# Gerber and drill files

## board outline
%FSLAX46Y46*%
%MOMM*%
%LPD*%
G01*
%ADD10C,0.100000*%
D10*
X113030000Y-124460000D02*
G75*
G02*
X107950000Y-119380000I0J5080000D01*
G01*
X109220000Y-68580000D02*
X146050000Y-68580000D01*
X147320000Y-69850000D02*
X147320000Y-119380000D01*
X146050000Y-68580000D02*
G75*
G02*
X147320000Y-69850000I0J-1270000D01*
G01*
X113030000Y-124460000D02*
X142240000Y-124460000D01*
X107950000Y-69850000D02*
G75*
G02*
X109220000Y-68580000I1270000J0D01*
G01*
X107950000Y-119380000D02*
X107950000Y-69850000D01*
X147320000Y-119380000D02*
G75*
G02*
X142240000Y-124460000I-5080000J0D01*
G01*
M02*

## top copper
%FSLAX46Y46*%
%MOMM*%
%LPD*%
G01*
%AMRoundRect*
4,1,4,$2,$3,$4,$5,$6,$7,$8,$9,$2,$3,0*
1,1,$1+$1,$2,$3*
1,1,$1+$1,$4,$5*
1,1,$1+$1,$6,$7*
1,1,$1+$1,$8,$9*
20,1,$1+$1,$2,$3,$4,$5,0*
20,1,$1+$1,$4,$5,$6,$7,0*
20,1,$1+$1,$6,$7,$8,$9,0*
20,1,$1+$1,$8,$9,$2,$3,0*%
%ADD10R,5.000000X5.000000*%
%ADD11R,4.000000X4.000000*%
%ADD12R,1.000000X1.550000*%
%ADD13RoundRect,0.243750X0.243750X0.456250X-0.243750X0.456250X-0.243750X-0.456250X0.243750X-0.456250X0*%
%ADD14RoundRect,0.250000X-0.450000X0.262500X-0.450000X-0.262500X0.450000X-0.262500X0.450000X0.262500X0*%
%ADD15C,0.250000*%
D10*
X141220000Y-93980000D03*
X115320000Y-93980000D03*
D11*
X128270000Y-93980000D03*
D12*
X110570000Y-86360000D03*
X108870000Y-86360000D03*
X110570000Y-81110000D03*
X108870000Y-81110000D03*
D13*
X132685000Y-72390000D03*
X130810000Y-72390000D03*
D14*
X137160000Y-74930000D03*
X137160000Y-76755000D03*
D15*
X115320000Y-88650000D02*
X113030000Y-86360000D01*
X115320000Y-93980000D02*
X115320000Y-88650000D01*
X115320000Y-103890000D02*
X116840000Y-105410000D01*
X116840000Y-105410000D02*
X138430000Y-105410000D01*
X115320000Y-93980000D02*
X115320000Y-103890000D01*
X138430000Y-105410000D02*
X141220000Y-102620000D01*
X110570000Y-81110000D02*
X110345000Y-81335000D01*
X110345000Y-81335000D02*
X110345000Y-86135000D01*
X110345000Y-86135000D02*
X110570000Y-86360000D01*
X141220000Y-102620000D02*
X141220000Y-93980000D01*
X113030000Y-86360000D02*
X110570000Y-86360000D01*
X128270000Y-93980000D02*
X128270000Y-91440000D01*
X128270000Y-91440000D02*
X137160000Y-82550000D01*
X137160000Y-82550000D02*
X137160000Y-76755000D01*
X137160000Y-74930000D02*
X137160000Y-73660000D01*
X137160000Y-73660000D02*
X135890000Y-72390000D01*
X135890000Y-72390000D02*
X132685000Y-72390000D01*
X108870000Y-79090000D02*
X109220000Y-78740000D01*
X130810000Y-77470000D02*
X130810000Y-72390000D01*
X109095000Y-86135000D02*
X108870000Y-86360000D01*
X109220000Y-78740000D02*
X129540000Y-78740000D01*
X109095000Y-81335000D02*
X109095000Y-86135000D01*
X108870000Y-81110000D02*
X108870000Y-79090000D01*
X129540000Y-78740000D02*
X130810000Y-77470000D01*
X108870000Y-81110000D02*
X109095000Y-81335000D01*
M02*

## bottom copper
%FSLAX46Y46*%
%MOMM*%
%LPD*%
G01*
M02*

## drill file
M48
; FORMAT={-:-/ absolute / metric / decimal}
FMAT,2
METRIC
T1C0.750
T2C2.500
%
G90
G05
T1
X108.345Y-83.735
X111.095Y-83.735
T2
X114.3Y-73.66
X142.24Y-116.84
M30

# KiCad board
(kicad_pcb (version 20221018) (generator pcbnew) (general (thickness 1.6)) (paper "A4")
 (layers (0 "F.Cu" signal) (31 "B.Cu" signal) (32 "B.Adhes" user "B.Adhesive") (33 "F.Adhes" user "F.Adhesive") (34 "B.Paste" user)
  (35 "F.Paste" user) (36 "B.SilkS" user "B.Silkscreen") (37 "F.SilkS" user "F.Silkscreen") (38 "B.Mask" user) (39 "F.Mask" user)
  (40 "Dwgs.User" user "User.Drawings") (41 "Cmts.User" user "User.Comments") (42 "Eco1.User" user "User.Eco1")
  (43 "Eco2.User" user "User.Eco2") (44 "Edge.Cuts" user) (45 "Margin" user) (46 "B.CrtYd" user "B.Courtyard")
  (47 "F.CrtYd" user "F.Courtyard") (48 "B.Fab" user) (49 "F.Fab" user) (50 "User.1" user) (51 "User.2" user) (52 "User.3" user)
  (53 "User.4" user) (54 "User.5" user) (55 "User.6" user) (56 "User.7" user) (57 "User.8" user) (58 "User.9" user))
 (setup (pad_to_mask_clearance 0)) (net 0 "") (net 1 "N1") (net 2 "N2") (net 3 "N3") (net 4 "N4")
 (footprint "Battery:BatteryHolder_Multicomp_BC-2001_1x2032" (layer "F.Cu") (at 128.27 93.98 180)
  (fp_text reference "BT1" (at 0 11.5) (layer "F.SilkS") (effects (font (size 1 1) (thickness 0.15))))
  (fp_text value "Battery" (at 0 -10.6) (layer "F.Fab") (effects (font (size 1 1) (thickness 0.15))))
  (pad "1" smd rect (at -12.95 0 180) (size 5 5) (layers "F.Cu" "F.Paste" "F.Mask") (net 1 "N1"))
  (pad "1" smd rect (at 12.95 0 180) (size 5 5) (layers "F.Cu" "F.Paste" "F.Mask") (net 1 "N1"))
  (pad "2" smd rect (at 0 0 180) (size 4 4) (layers "F.Cu" "F.Paste" "F.Mask") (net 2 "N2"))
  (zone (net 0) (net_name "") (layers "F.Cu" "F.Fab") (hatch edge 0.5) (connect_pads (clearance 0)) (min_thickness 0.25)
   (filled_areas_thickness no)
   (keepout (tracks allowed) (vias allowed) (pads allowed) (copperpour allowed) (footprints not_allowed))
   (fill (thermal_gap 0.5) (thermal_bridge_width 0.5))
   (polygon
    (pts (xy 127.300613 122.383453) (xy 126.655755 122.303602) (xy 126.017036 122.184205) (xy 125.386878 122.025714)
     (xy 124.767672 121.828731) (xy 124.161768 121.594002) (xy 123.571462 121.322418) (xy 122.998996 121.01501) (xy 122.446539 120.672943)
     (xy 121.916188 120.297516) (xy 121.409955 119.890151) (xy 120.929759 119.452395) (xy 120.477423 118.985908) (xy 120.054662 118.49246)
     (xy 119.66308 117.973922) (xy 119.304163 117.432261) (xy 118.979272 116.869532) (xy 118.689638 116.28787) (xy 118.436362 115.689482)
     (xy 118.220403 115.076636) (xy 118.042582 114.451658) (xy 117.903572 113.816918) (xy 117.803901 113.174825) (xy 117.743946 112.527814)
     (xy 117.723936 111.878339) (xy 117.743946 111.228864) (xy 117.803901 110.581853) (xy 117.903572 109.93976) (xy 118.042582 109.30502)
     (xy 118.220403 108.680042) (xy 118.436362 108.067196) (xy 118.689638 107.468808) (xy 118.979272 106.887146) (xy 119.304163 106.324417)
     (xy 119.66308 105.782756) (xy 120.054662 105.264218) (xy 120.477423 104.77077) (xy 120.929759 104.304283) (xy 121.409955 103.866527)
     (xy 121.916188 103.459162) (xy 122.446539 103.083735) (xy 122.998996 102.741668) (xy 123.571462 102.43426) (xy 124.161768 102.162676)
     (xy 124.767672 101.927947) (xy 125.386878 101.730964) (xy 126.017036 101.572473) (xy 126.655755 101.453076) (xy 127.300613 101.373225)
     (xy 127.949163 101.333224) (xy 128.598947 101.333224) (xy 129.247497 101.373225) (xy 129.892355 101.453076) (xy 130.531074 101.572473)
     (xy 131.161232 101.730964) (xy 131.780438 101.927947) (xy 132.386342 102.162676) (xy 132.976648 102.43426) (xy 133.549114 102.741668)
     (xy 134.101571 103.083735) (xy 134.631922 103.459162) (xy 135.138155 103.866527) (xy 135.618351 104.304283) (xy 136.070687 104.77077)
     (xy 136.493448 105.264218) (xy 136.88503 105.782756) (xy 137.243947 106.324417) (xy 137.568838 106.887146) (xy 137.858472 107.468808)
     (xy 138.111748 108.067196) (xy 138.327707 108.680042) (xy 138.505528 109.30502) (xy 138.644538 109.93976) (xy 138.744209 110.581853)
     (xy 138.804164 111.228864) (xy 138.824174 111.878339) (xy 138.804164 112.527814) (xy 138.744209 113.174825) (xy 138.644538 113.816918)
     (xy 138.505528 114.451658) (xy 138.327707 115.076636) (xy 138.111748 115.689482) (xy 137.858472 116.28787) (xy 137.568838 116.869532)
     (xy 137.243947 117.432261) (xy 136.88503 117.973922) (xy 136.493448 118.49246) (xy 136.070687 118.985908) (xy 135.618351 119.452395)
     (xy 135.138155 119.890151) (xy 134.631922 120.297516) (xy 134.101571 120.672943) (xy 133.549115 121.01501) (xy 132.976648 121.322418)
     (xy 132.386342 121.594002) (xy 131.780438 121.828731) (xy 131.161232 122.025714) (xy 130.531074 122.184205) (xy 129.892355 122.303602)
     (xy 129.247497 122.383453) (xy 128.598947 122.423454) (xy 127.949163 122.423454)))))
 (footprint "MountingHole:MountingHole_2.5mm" (layer "F.Cu") (at 142.24 116.84)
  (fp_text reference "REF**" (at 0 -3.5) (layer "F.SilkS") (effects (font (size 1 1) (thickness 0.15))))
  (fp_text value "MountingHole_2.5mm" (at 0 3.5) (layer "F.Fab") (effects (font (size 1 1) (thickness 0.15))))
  (pad "" np_thru_hole circle (at 0 0) (size 2.5 2.5) (drill 2.5) (layers "*.Cu" "*.Mask")))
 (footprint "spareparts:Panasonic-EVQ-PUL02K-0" (layer "F.Cu") (at 109.22 83.735 -90)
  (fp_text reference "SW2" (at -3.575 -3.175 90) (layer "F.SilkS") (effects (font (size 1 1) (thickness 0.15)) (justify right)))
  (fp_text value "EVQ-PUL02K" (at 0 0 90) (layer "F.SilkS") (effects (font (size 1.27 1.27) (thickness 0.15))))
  (pad "" np_thru_hole circle (at 0 -1.875 270) (size 0.75 0.75) (drill 0.75) (layers "*.Cu" "*.Mask"))
  (pad "" np_thru_hole circle (at 0 0.875 270) (size 0.75 0.75) (drill 0.75) (layers "*.Cu" "*.Mask"))
  (pad "1" smd rect (at 2.625 -1.35 270) (size 1.55 1) (layers "F.Cu" "F.Paste" "F.Mask") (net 1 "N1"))
  (pad "2" smd rect (at 2.625 0.35 270) (size 1.55 1) (layers "F.Cu" "F.Paste" "F.Mask") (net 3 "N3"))
  (pad "3" smd rect (at -2.625 -1.35 270) (size 1.55 1) (layers "F.Cu" "F.Paste" "F.Mask") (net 1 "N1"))
  (pad "4" smd rect (at -2.625 0.35 270) (size 1.55 1) (layers "F.Cu" "F.Paste" "F.Mask") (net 3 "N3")))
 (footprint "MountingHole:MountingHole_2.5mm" (layer "F.Cu") (at 114.3 73.66)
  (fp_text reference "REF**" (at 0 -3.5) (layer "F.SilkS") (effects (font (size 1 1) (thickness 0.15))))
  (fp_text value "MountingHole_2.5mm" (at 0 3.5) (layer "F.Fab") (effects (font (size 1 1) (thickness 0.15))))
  (pad "" np_thru_hole circle (at 0 0) (size 2.5 2.5) (drill 2.5) (layers "*.Cu" "*.Mask")))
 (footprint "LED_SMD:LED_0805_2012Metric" (layer "F.Cu") (at 131.7475 72.39 180)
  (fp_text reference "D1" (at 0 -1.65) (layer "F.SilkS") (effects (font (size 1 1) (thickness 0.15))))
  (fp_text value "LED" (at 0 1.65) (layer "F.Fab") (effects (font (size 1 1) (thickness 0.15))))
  (pad "1" smd roundrect (at -0.9375 0 180) (size 0.975 1.4) (layers "F.Cu" "F.Paste" "F.Mask") (roundrect_rratio 0.25) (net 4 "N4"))
  (pad "2" smd roundrect (at 0.9375 0 180) (size 0.975 1.4) (layers "F.Cu" "F.Paste" "F.Mask") (roundrect_rratio 0.25) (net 3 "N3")))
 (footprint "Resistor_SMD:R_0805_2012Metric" (layer "F.Cu") (at 137.16 75.8425 -90)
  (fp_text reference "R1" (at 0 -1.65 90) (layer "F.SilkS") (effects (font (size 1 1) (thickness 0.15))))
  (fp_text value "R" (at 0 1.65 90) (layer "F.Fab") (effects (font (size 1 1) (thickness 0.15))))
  (pad "1" smd roundrect (at -0.9125 0 270) (size 1.025 1.4) (layers "F.Cu" "F.Paste" "F.Mask") (roundrect_rratio 0.243902) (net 4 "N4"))
  (pad "2" smd roundrect (at 0.9125 0 270) (size 1.025 1.4) (layers "F.Cu" "F.Paste" "F.Mask") (roundrect_rratio 0.243902) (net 2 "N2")))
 (gr_arc (start 113.03 124.46) (mid 109.437898 122.972102) (end 107.95 119.38) (stroke (width 0.1) (type default)) (layer "Edge.Cuts"))
 (gr_line (start 109.22 68.58) (end 146.05 68.58) (stroke (width 0.1) (type default)) (layer "Edge.Cuts"))
 (gr_line (start 147.32 69.85) (end 147.32 119.38) (stroke (width 0.1) (type default)) (layer "Edge.Cuts"))
 (gr_arc (start 146.05 68.58) (mid 146.948026 68.951974) (end 147.32 69.85) (stroke (width 0.1) (type default)) (layer "Edge.Cuts"))
 (gr_line (start 113.03 124.46) (end 142.24 124.46) (stroke (width 0.1) (type default)) (layer "Edge.Cuts"))
 (gr_arc (start 107.95 69.85) (mid 108.321974 68.951974) (end 109.22 68.58) (stroke (width 0.1) (type default)) (layer "Edge.Cuts"))
 (gr_line (start 107.95 119.38) (end 107.95 69.85) (stroke (width 0.1) (type default)) (layer "Edge.Cuts"))
 (gr_arc (start 147.32 119.38) (mid 145.832102 122.972102) (end 142.24 124.46) (stroke (width 0.1) (type default)) (layer "Edge.Cuts"))
 (segment (start 115.32 88.65) (end 113.03 86.36) (width 0.25) (layer "F.Cu") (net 1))
 (segment (start 115.32 93.98) (end 115.32 88.65) (width 0.25) (layer "F.Cu") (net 1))
 (segment (start 115.32 103.89) (end 116.84 105.41) (width 0.25) (layer "F.Cu") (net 1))
 (segment (start 116.84 105.41) (end 138.43 105.41) (width 0.25) (layer "F.Cu") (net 1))
 (segment (start 115.32 93.98) (end 115.32 103.89) (width 0.25) (layer "F.Cu") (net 1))
 (segment (start 138.43 105.41) (end 141.22 102.62) (width 0.25) (layer "F.Cu") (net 1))
 (segment (start 110.57 81.11) (end 110.345 81.335) (width 0.25) (layer "F.Cu") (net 1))
 (segment (start 110.345 81.335) (end 110.345 86.135) (width 0.25) (layer "F.Cu") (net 1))
 (segment (start 110.345 86.135) (end 110.57 86.36) (width 0.25) (layer "F.Cu") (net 1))
 (segment (start 141.22 102.62) (end 141.22 93.98) (width 0.25) (layer "F.Cu") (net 1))
 (segment (start 113.03 86.36) (end 110.57 86.36) (width 0.25) (layer "F.Cu") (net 1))
 (segment (start 128.27 93.98) (end 128.27 91.44) (width 0.25) (layer "F.Cu") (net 2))
 (segment (start 128.27 91.44) (end 137.16 82.55) (width 0.25) (layer "F.Cu") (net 2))
 (segment (start 137.16 82.55) (end 137.16 76.755) (width 0.25) (layer "F.Cu") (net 2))
 (segment (start 137.16 74.93) (end 137.16 73.66) (width 0.25) (layer "F.Cu") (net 4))
 (segment (start 137.16 73.66) (end 135.89 72.39) (width 0.25) (layer "F.Cu") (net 4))
 (segment (start 135.89 72.39) (end 132.685 72.39) (width 0.25) (layer "F.Cu") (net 4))
 (segment (start 108.87 79.09) (end 109.22 78.74) (width 0.25) (layer "F.Cu") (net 3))
 (segment (start 130.81 77.47) (end 130.81 72.39) (width 0.25) (layer "F.Cu") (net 3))
 (segment (start 109.095 86.135) (end 108.87 86.36) (width 0.25) (layer "F.Cu") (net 3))
 (segment (start 109.22 78.74) (end 129.54 78.74) (width 0.25) (layer "F.Cu") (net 3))
 (segment (start 109.095 81.335) (end 109.095 86.135) (width 0.25) (layer "F.Cu") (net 3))
 (segment (start 108.87 81.11) (end 108.87 79.09) (width 0.25) (layer "F.Cu") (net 3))
 (segment (start 129.54 78.74) (end 130.81 77.47) (width 0.25) (layer "F.Cu") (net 3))
 (segment (start 108.87 81.11) (end 109.095 81.335) (width 0.25) (layer "F.Cu") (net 3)))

